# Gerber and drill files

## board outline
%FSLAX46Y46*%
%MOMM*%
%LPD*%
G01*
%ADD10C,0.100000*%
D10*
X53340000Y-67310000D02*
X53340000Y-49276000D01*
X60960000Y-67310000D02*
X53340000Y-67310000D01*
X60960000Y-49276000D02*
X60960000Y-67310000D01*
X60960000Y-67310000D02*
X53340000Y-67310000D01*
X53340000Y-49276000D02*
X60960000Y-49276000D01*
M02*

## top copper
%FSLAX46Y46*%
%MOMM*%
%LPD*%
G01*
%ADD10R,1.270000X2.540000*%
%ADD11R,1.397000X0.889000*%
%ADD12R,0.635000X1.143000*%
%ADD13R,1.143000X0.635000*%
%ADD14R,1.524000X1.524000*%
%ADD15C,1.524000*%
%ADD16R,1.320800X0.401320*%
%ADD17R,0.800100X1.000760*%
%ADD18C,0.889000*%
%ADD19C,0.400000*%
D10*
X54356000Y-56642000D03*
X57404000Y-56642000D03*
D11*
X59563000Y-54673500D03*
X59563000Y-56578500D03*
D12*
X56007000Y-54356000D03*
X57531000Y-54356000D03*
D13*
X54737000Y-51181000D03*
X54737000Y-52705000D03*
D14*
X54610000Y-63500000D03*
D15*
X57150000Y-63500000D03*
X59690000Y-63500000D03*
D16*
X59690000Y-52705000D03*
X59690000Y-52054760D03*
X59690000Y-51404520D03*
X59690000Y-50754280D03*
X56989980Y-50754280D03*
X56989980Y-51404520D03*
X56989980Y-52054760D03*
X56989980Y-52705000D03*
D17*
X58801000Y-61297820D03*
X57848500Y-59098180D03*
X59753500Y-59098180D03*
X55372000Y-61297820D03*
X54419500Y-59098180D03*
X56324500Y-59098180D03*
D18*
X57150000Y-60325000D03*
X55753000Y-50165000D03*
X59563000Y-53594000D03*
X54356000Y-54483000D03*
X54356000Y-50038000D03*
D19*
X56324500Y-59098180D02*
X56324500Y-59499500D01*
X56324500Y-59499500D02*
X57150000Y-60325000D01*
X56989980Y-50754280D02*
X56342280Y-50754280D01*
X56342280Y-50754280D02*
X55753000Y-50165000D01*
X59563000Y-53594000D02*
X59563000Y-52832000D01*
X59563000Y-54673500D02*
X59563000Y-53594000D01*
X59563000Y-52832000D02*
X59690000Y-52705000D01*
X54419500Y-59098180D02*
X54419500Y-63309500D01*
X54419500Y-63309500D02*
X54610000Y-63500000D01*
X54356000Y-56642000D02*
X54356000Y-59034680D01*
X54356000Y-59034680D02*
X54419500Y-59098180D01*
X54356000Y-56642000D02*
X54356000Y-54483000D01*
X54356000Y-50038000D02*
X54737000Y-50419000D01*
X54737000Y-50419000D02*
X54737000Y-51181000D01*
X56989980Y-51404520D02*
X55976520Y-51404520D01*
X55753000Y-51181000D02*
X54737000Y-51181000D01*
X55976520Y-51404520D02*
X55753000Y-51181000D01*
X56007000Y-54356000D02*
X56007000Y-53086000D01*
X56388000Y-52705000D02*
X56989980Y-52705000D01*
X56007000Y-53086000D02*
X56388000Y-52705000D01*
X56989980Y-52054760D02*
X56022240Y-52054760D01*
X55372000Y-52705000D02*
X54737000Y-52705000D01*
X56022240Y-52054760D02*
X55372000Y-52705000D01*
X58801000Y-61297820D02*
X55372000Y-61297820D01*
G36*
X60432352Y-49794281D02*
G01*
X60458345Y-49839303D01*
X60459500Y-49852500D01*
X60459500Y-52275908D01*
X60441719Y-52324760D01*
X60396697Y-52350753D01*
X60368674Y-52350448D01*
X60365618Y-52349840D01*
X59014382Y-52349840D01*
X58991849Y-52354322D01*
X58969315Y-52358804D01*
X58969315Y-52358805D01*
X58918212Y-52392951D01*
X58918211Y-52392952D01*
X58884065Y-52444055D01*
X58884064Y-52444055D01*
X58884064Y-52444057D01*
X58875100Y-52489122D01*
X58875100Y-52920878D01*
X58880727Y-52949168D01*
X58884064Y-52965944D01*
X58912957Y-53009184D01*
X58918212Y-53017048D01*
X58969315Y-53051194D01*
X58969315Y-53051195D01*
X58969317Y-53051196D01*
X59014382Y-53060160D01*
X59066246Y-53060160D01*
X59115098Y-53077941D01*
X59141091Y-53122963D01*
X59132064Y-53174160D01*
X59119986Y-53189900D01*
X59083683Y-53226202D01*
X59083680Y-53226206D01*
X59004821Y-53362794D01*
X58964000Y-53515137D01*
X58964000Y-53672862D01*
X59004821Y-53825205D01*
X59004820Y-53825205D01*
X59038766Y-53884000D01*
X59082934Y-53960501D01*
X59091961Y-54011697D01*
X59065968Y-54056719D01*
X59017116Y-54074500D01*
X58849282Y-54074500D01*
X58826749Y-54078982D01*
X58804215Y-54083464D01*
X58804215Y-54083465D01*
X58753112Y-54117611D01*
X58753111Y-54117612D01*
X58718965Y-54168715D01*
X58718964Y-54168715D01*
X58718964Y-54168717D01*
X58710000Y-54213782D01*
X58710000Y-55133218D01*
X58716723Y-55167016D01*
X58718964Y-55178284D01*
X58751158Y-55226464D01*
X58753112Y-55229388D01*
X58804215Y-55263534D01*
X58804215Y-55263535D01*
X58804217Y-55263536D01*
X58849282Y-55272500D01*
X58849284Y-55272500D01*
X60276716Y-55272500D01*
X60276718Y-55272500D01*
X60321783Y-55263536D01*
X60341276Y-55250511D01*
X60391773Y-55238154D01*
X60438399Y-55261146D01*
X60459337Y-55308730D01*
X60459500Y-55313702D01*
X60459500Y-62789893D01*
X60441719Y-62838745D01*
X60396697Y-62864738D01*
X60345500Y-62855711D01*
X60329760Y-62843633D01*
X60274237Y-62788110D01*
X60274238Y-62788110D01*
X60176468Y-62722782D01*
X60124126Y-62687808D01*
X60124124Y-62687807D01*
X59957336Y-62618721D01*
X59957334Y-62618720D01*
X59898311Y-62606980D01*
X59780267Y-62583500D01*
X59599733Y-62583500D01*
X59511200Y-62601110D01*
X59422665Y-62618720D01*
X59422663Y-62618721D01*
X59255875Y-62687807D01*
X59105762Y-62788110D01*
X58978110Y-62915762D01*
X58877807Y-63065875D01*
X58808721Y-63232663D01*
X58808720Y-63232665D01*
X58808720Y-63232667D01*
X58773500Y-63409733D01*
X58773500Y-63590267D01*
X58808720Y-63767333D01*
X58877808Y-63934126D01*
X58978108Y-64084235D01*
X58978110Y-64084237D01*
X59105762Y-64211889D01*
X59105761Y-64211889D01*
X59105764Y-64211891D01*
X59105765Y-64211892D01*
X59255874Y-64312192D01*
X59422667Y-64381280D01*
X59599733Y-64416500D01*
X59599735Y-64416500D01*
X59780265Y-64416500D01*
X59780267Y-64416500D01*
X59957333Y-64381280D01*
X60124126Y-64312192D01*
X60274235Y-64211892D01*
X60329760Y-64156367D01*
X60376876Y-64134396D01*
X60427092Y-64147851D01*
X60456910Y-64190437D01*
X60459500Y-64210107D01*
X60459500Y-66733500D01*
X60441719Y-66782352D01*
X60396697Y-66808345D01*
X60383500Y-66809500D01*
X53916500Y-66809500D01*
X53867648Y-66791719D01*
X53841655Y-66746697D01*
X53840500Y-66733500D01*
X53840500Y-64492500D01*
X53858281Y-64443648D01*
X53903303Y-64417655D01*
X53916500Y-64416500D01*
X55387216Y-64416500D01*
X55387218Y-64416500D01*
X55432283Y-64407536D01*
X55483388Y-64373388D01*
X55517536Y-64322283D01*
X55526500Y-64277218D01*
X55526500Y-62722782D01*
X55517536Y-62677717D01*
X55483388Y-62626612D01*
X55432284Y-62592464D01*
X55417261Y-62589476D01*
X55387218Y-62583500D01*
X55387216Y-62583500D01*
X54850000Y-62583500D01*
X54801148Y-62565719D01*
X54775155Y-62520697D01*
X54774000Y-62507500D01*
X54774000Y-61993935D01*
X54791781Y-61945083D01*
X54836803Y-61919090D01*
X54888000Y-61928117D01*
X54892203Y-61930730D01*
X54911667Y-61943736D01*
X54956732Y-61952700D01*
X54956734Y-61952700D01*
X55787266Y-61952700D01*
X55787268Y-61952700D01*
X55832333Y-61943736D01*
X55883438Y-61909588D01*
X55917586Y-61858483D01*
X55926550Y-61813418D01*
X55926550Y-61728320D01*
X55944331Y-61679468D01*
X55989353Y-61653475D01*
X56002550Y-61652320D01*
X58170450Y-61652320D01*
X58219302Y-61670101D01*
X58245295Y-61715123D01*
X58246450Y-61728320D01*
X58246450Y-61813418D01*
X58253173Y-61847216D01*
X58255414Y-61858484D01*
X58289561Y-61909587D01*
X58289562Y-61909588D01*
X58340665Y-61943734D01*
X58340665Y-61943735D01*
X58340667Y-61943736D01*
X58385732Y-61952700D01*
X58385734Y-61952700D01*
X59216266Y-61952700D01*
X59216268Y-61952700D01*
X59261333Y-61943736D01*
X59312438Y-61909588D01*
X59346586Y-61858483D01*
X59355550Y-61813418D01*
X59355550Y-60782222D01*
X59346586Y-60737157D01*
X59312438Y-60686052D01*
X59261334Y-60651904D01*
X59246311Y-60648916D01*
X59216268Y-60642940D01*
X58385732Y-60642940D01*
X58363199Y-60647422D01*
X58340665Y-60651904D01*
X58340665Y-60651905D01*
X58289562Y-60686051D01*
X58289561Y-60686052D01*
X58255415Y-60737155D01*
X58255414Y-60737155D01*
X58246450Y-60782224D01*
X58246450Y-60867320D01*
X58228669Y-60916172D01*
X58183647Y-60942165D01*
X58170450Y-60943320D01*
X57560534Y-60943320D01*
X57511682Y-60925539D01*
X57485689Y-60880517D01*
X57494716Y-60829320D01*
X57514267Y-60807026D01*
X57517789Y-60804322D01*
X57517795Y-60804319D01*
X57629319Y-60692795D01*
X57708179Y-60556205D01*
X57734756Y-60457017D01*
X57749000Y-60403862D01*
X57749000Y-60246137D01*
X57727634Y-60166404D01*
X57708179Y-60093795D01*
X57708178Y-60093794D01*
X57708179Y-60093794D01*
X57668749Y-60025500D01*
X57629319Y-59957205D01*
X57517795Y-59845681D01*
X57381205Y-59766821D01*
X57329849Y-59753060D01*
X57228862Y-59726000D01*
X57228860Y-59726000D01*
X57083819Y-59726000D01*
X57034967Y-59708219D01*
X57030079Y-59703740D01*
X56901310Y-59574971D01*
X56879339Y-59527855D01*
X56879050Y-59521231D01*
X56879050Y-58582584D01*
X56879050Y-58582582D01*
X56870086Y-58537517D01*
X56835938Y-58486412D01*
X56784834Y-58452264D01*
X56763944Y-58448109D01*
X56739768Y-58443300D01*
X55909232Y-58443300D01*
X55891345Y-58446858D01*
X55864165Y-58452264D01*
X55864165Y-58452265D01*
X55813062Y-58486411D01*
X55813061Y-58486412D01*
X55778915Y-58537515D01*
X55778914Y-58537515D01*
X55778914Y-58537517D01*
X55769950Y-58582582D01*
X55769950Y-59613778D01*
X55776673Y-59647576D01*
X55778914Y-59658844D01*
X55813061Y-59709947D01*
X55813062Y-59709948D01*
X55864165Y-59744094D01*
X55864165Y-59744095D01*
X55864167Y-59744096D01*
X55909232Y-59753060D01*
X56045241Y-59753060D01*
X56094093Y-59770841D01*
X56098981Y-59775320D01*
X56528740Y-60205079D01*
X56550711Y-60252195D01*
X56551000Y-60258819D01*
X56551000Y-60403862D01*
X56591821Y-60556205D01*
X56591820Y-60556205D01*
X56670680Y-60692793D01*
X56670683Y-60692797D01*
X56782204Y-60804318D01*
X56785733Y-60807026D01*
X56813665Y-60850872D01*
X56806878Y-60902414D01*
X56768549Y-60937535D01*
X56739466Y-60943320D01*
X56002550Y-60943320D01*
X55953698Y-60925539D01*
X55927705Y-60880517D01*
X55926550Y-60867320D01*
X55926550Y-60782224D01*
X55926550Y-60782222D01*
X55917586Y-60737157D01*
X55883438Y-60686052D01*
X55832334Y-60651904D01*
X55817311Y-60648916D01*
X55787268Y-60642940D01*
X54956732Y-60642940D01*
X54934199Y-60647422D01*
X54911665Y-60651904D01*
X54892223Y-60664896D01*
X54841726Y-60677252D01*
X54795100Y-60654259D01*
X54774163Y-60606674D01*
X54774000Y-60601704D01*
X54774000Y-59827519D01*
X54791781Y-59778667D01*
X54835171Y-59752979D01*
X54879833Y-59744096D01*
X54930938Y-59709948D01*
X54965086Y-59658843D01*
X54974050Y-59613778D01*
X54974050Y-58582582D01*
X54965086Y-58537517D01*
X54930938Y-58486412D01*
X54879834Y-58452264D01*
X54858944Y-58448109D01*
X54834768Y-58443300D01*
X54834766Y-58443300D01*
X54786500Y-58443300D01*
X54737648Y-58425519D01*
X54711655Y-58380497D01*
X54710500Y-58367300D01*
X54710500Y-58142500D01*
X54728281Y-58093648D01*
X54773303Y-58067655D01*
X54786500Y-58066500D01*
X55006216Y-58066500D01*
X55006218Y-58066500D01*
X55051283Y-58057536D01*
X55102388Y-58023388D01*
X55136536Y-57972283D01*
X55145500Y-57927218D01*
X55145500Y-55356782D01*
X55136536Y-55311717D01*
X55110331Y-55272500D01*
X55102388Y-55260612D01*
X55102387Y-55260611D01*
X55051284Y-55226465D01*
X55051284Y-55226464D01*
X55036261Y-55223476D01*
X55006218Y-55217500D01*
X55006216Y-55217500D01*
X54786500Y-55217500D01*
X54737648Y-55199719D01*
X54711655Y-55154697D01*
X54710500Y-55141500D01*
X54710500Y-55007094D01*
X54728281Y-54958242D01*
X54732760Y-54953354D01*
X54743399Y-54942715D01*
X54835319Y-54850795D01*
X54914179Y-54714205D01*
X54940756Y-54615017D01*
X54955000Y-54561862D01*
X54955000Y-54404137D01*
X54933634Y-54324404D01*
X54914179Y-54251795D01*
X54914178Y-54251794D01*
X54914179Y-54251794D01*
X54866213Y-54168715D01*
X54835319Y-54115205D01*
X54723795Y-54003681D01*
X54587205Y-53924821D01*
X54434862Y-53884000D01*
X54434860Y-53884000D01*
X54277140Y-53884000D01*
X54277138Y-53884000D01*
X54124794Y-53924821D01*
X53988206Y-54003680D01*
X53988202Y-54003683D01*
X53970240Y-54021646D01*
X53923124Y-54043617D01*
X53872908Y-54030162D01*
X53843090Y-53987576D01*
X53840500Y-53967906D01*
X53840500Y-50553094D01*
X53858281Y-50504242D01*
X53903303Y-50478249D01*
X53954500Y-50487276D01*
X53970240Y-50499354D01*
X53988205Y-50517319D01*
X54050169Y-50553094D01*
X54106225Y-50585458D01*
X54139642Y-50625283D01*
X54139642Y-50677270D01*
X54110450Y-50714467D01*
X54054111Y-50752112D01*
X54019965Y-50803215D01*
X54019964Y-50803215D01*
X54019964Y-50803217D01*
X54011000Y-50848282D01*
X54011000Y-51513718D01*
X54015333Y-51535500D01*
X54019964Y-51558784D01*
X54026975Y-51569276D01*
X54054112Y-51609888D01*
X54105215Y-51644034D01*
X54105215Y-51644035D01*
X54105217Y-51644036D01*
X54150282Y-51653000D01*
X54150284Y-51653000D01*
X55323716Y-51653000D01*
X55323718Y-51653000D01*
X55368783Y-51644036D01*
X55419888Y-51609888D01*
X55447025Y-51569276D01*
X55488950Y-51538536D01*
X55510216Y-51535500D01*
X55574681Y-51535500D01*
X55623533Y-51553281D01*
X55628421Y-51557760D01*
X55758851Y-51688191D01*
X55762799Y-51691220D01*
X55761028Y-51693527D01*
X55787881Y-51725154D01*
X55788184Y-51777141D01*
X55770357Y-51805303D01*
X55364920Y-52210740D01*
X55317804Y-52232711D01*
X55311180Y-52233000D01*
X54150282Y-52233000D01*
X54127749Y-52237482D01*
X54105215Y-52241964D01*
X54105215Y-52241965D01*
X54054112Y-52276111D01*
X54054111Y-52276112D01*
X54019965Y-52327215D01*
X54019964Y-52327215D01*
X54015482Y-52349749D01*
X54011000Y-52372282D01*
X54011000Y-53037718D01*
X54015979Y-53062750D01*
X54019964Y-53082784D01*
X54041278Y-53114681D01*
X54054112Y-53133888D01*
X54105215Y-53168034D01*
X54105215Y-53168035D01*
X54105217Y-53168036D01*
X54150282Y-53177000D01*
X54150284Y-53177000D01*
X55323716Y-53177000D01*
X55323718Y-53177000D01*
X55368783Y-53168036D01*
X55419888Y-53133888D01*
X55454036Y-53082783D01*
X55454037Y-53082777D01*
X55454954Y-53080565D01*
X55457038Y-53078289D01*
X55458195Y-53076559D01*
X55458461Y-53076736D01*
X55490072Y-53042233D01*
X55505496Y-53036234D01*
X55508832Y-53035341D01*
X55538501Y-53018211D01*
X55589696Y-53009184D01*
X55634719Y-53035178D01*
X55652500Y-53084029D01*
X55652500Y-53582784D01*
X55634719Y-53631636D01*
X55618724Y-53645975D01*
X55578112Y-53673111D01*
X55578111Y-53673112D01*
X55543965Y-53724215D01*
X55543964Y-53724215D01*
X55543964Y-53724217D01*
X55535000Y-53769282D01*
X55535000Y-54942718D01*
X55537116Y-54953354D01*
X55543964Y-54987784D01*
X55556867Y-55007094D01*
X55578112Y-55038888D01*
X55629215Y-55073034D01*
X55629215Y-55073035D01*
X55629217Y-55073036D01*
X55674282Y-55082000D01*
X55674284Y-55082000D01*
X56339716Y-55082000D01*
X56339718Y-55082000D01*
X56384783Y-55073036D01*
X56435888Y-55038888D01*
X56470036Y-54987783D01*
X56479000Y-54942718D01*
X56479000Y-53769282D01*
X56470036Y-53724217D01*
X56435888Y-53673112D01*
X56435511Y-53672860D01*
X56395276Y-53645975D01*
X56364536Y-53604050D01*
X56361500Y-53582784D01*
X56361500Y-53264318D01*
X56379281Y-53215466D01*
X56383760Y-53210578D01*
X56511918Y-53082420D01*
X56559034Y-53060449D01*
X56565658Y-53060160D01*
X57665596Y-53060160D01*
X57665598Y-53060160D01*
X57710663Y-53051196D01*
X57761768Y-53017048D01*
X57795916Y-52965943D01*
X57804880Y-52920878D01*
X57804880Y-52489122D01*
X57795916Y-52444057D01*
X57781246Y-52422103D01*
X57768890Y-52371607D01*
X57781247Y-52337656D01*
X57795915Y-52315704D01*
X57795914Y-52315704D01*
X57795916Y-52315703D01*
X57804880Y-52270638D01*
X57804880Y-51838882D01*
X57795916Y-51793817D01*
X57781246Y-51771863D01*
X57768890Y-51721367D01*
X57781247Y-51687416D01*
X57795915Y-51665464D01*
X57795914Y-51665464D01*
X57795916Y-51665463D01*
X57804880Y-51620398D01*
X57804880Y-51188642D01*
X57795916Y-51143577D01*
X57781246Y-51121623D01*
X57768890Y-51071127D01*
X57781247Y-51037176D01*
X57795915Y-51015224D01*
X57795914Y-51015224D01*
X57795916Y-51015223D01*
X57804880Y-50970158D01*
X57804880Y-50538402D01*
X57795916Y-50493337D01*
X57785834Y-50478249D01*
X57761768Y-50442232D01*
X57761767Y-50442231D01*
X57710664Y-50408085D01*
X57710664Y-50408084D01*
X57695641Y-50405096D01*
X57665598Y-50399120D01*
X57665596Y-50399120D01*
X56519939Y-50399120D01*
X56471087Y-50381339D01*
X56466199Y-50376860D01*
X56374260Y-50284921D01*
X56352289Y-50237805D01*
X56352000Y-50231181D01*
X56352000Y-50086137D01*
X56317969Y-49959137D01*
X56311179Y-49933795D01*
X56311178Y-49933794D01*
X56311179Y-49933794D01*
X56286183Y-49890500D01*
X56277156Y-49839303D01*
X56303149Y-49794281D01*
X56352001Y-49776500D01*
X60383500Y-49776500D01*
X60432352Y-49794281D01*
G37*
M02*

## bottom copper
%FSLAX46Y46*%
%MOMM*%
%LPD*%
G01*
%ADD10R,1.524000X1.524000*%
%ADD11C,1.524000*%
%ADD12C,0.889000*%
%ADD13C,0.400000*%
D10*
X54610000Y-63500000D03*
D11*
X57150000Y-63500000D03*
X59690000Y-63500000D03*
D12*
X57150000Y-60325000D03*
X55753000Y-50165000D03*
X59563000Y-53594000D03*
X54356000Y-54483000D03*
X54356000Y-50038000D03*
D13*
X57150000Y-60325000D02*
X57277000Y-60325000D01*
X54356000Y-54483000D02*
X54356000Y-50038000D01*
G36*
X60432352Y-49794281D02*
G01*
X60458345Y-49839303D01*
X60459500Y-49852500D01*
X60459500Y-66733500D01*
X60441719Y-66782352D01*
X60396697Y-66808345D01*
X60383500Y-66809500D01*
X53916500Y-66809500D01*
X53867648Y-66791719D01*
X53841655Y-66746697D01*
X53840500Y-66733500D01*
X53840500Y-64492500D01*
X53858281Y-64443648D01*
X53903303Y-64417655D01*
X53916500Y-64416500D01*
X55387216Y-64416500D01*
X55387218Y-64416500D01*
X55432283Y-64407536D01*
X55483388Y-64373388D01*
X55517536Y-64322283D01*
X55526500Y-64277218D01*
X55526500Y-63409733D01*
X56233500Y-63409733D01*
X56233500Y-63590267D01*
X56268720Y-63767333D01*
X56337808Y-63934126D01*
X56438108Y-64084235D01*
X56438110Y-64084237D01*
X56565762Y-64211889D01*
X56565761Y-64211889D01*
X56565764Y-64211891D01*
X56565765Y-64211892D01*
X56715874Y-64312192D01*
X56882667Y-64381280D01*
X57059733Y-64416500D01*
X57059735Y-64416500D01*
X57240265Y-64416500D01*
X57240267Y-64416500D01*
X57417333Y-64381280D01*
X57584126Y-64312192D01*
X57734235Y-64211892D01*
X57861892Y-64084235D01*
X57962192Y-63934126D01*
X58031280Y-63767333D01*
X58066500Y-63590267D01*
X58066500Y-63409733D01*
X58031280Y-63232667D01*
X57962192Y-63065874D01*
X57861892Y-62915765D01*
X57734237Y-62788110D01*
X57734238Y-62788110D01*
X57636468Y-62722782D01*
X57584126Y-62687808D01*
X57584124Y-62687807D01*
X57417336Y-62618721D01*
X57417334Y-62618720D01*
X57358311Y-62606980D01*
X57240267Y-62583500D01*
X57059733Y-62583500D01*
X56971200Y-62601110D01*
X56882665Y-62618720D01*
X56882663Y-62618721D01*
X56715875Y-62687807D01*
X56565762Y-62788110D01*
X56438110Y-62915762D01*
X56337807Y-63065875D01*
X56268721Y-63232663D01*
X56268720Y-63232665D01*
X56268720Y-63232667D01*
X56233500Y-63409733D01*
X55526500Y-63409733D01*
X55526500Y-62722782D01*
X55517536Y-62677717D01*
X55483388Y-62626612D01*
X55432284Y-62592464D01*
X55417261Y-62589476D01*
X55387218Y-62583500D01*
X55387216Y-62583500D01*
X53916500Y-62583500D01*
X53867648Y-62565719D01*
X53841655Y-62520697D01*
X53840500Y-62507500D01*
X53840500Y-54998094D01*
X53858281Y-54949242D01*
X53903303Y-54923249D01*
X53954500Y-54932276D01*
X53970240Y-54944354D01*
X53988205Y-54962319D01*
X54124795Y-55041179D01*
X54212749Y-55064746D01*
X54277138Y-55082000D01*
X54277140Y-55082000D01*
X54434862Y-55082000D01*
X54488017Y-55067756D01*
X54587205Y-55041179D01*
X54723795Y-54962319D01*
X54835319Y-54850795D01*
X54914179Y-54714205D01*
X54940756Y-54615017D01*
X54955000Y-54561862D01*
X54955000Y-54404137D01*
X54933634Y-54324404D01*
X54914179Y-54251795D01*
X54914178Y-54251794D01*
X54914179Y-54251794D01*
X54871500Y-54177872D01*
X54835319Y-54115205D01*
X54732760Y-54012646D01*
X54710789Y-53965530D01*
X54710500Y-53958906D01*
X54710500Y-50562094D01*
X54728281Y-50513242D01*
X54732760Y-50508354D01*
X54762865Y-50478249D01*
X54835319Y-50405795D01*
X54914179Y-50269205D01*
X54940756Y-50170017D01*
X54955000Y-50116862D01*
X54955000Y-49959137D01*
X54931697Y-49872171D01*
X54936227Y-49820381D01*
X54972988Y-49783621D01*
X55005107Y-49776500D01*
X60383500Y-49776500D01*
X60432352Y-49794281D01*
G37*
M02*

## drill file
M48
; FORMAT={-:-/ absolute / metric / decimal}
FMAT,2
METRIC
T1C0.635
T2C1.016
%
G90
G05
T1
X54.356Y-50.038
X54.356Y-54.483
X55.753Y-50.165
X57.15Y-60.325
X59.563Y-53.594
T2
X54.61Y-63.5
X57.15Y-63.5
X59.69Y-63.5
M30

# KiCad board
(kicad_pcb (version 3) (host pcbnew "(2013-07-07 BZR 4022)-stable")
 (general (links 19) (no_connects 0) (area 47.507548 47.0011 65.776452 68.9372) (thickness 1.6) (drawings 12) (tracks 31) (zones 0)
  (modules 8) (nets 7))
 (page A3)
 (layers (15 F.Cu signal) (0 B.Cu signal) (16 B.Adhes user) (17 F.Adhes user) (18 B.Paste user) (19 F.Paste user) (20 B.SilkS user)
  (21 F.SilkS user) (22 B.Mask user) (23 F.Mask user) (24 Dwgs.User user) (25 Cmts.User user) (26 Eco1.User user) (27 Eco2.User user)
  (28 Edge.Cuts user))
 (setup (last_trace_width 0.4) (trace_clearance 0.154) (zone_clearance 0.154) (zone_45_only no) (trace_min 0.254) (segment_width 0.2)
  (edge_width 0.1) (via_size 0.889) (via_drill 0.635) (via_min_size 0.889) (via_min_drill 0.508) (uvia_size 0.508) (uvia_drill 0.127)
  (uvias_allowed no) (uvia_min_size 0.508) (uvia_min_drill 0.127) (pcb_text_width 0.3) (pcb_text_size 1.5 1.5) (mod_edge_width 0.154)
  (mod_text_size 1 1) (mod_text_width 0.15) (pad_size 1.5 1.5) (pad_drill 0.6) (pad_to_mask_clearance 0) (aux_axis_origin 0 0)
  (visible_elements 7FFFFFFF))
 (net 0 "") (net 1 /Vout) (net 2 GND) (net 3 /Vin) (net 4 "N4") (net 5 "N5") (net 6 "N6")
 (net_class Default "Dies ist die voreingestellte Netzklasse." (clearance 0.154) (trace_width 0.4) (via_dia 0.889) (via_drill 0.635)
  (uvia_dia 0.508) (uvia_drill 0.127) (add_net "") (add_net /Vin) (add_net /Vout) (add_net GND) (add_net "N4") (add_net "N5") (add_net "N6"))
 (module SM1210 (layer F.Cu) (at 55.88 56.642)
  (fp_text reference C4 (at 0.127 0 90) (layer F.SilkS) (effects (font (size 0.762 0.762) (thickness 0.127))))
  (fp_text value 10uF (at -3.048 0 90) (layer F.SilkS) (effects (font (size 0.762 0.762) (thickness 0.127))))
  (pad 1 smd rect (at -1.524 0) (size 1.27 2.54) (layers F.Cu F.Paste F.Mask) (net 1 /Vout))
  (pad 2 smd rect (at 1.524 0) (size 1.27 2.54) (layers F.Cu F.Paste F.Mask) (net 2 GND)))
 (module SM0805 (layer F.Cu) (at 59.563 55.626 270)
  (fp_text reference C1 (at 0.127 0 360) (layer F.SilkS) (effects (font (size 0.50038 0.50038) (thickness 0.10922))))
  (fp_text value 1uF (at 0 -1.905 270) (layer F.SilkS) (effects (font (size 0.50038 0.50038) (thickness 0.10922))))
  (pad 1 smd rect (at -0.9525 0 270) (size 0.889 1.397) (layers F.Cu F.Paste F.Mask) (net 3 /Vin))
  (pad 2 smd rect (at 0.9525 0 270) (size 0.889 1.397) (layers F.Cu F.Paste F.Mask) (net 2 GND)))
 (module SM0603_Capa (layer F.Cu) (at 56.769 54.356)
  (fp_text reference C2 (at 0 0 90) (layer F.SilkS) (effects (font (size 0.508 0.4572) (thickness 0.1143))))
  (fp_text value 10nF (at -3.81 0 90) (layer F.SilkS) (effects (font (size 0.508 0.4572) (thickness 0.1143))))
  (pad 1 smd rect (at -0.762 0) (size 0.635 1.143) (layers F.Cu F.Paste F.Mask) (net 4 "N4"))
  (pad 2 smd rect (at 0.762 0) (size 0.635 1.143) (layers F.Cu F.Paste F.Mask) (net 2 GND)))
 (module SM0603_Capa (layer F.Cu) (at 54.737 51.943 270)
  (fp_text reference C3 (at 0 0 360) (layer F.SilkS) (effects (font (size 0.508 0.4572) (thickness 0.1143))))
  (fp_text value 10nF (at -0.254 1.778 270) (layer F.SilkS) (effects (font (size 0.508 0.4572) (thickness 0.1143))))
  (pad 1 smd rect (at -0.762 0 270) (size 0.635 1.143) (layers F.Cu F.Paste F.Mask) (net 1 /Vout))
  (pad 2 smd rect (at 0.762 0 270) (size 0.635 1.143) (layers F.Cu F.Paste F.Mask) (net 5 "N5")))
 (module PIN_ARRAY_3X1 (layer F.Cu) (at 57.15 63.5)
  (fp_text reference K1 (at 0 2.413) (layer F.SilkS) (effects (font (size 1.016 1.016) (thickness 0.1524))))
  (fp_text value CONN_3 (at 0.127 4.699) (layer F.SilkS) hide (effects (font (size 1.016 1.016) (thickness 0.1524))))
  (pad 1 thru_hole rect (at -2.54 0) (size 1.524 1.524) (drill 1.016) (layers *.Cu *.Mask F.SilkS) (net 1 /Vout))
  (pad 2 thru_hole circle (at 0 0) (size 1.524 1.524) (drill 1.016) (layers *.Cu *.Mask F.SilkS) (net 2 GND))
  (pad 3 thru_hole circle (at 2.54 0) (size 1.524 1.524) (drill 1.016) (layers *.Cu *.Mask F.SilkS) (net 3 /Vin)))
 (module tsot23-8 (layer F.Cu) (at 59.69 52.705 90)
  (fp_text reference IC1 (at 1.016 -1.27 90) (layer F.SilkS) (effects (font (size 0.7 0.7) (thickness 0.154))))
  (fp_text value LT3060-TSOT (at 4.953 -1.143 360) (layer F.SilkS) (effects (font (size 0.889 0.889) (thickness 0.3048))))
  (pad 1 smd rect (at 0 0 90) (size 0.40132 1.3208) (layers F.Cu F.Paste F.Mask) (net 3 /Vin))
  (pad 2 smd rect (at 0.65024 0 90) (size 0.40132 1.3208) (layers F.Cu F.Paste F.Mask) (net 2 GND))
  (pad 3 smd rect (at 1.30048 0 90) (size 0.40132 1.3208) (layers F.Cu F.Paste F.Mask) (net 2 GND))
  (pad 4 smd rect (at 1.95072 0 90) (size 0.40132 1.3208) (layers F.Cu F.Paste F.Mask) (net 2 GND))
  (pad 5 smd rect (at 1.95072 -2.70002 270) (size 0.40132 1.3208) (layers F.Cu F.Paste F.Mask) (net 3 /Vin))
  (pad 6 smd rect (at 1.30048 -2.70002 270) (size 0.40132 1.3208) (layers F.Cu F.Paste F.Mask) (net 1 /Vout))
  (pad 7 smd rect (at 0.65024 -2.70002 270) (size 0.40132 1.3208) (layers F.Cu F.Paste F.Mask) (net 5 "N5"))
  (pad 8 smd rect (at 0 -2.70002 270) (size 0.40132 1.3208) (layers F.Cu F.Paste F.Mask) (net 4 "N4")))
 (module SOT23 (layer F.Cu) (at 58.801 60.198 180)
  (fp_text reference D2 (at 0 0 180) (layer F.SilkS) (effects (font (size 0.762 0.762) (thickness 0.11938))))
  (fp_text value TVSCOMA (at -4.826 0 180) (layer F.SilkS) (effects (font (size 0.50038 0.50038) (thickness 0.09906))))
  (pad 3 smd rect (at 0 -1.09982 180) (size 0.8001 1.00076) (layers F.Cu F.Paste F.Mask) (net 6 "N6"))
  (pad 2 smd rect (at 0.9525 1.09982 180) (size 0.8001 1.00076) (layers F.Cu F.Paste F.Mask) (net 2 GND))
  (pad 1 smd rect (at -0.9525 1.09982 180) (size 0.8001 1.00076) (layers F.Cu F.Paste F.Mask) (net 2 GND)))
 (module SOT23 (layer F.Cu) (at 55.372 60.198 180)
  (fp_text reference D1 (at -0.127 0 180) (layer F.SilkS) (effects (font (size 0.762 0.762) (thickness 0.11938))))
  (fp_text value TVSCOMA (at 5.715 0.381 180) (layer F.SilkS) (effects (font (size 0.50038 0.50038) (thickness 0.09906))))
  (pad 3 smd rect (at 0 -1.09982 180) (size 0.8001 1.00076) (layers F.Cu F.Paste F.Mask) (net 6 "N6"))
  (pad 2 smd rect (at 0.9525 1.09982 180) (size 0.8001 1.00076) (layers F.Cu F.Paste F.Mask) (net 1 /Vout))
  (pad 1 smd rect (at -0.9525 1.09982 180) (size 0.8001 1.00076) (layers F.Cu F.Paste F.Mask) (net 3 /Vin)))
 (gr_line (start 53.34 67.31) (end 53.34 49.276) (angle 90) (layer Edge.Cuts) (width 0.1))
 (gr_line (start 60.96 67.31) (end 53.34 67.31) (angle 90) (layer Edge.Cuts) (width 0.1))
 (gr_line (start 60.96 49.276) (end 60.96 67.31) (angle 90) (layer Edge.Cuts) (width 0.1))
 (gr_line (start 60.96 67.31) (end 53.34 67.31) (angle 90) (layer Edge.Cuts) (width 0.1))
 (gr_line (start 53.34 49.276) (end 60.96 49.276) (angle 90) (layer Edge.Cuts) (width 0.1))
 (segment (start 56.3245 59.09818) (end 56.3245 59.4995) (width 0.4) (layer F.Cu) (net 3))
 (segment (start 57.15 60.325) (end 57.277 60.325) (width 0.4) (layer B.Cu) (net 3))
 (via (at 57.15 60.325) (size 0.889) (layers F.Cu B.Cu) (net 3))
 (segment (start 56.3245 59.4995) (end 57.15 60.325) (width 0.4) (layer F.Cu) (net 3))
 (segment (start 56.98998 50.75428) (end 56.34228 50.75428) (width 0.4) (layer F.Cu) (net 3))
 (via (at 55.753 50.165) (size 0.889) (layers F.Cu B.Cu) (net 3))
 (segment (start 56.34228 50.75428) (end 55.753 50.165) (width 0.4) (layer F.Cu) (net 3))
 (segment (start 59.563 53.594) (end 59.563 52.832) (width 0.4) (layer F.Cu) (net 3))
 (via (at 59.563 53.594) (size 0.889) (layers F.Cu B.Cu) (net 3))
 (segment (start 59.563 54.6735) (end 59.563 53.594) (width 0.4) (layer F.Cu) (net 3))
 (segment (start 59.563 52.832) (end 59.69 52.705) (width 0.4) (layer F.Cu) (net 3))
 (segment (start 54.4195 59.09818) (end 54.4195 63.3095) (width 0.4) (layer F.Cu) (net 1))
 (segment (start 54.4195 63.3095) (end 54.61 63.5) (width 0.4) (layer F.Cu) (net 1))
 (segment (start 54.356 56.642) (end 54.356 59.03468) (width 0.4) (layer F.Cu) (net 1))
 (segment (start 54.356 59.03468) (end 54.4195 59.09818) (width 0.4) (layer F.Cu) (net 1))
 (segment (start 54.356 56.642) (end 54.356 54.483) (width 0.4) (layer F.Cu) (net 1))
 (via (at 54.356 54.483) (size 0.889) (layers F.Cu B.Cu) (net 1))
 (segment (start 54.356 54.483) (end 54.356 50.038) (width 0.4) (layer B.Cu) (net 1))
 (via (at 54.356 50.038) (size 0.889) (layers F.Cu B.Cu) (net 1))
 (segment (start 54.356 50.038) (end 54.737 50.419) (width 0.4) (layer F.Cu) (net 1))
 (segment (start 54.737 50.419) (end 54.737 51.181) (width 0.4) (layer F.Cu) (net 1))
 (segment (start 56.98998 51.40452) (end 55.97652 51.40452) (width 0.4) (layer F.Cu) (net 1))
 (segment (start 55.753 51.181) (end 54.737 51.181) (width 0.4) (layer F.Cu) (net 1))
 (segment (start 55.97652 51.40452) (end 55.753 51.181) (width 0.4) (layer F.Cu) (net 1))
 (segment (start 56.007 54.356) (end 56.007 53.086) (width 0.4) (layer F.Cu) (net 4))
 (segment (start 56.388 52.705) (end 56.98998 52.705) (width 0.4) (layer F.Cu) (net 4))
 (segment (start 56.007 53.086) (end 56.388 52.705) (width 0.4) (layer F.Cu) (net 4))
 (segment (start 56.98998 52.05476) (end 56.02224 52.05476) (width 0.4) (layer F.Cu) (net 5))
 (segment (start 55.372 52.705) (end 54.737 52.705) (width 0.4) (layer F.Cu) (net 5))
 (segment (start 56.02224 52.05476) (end 55.372 52.705) (width 0.4) (layer F.Cu) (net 5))
 (segment (start 58.801 61.29782) (end 55.372 61.29782) (width 0.4) (layer F.Cu) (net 6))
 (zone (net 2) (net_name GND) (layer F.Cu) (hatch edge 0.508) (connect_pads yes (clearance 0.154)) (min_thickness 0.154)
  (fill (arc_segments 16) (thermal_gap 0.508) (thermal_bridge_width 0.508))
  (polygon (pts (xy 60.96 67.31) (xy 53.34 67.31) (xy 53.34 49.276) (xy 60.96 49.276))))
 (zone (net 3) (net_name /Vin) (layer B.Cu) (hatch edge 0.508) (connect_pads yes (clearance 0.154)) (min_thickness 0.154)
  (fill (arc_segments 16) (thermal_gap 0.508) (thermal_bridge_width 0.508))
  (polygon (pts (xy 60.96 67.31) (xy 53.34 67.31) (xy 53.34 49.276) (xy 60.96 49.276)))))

